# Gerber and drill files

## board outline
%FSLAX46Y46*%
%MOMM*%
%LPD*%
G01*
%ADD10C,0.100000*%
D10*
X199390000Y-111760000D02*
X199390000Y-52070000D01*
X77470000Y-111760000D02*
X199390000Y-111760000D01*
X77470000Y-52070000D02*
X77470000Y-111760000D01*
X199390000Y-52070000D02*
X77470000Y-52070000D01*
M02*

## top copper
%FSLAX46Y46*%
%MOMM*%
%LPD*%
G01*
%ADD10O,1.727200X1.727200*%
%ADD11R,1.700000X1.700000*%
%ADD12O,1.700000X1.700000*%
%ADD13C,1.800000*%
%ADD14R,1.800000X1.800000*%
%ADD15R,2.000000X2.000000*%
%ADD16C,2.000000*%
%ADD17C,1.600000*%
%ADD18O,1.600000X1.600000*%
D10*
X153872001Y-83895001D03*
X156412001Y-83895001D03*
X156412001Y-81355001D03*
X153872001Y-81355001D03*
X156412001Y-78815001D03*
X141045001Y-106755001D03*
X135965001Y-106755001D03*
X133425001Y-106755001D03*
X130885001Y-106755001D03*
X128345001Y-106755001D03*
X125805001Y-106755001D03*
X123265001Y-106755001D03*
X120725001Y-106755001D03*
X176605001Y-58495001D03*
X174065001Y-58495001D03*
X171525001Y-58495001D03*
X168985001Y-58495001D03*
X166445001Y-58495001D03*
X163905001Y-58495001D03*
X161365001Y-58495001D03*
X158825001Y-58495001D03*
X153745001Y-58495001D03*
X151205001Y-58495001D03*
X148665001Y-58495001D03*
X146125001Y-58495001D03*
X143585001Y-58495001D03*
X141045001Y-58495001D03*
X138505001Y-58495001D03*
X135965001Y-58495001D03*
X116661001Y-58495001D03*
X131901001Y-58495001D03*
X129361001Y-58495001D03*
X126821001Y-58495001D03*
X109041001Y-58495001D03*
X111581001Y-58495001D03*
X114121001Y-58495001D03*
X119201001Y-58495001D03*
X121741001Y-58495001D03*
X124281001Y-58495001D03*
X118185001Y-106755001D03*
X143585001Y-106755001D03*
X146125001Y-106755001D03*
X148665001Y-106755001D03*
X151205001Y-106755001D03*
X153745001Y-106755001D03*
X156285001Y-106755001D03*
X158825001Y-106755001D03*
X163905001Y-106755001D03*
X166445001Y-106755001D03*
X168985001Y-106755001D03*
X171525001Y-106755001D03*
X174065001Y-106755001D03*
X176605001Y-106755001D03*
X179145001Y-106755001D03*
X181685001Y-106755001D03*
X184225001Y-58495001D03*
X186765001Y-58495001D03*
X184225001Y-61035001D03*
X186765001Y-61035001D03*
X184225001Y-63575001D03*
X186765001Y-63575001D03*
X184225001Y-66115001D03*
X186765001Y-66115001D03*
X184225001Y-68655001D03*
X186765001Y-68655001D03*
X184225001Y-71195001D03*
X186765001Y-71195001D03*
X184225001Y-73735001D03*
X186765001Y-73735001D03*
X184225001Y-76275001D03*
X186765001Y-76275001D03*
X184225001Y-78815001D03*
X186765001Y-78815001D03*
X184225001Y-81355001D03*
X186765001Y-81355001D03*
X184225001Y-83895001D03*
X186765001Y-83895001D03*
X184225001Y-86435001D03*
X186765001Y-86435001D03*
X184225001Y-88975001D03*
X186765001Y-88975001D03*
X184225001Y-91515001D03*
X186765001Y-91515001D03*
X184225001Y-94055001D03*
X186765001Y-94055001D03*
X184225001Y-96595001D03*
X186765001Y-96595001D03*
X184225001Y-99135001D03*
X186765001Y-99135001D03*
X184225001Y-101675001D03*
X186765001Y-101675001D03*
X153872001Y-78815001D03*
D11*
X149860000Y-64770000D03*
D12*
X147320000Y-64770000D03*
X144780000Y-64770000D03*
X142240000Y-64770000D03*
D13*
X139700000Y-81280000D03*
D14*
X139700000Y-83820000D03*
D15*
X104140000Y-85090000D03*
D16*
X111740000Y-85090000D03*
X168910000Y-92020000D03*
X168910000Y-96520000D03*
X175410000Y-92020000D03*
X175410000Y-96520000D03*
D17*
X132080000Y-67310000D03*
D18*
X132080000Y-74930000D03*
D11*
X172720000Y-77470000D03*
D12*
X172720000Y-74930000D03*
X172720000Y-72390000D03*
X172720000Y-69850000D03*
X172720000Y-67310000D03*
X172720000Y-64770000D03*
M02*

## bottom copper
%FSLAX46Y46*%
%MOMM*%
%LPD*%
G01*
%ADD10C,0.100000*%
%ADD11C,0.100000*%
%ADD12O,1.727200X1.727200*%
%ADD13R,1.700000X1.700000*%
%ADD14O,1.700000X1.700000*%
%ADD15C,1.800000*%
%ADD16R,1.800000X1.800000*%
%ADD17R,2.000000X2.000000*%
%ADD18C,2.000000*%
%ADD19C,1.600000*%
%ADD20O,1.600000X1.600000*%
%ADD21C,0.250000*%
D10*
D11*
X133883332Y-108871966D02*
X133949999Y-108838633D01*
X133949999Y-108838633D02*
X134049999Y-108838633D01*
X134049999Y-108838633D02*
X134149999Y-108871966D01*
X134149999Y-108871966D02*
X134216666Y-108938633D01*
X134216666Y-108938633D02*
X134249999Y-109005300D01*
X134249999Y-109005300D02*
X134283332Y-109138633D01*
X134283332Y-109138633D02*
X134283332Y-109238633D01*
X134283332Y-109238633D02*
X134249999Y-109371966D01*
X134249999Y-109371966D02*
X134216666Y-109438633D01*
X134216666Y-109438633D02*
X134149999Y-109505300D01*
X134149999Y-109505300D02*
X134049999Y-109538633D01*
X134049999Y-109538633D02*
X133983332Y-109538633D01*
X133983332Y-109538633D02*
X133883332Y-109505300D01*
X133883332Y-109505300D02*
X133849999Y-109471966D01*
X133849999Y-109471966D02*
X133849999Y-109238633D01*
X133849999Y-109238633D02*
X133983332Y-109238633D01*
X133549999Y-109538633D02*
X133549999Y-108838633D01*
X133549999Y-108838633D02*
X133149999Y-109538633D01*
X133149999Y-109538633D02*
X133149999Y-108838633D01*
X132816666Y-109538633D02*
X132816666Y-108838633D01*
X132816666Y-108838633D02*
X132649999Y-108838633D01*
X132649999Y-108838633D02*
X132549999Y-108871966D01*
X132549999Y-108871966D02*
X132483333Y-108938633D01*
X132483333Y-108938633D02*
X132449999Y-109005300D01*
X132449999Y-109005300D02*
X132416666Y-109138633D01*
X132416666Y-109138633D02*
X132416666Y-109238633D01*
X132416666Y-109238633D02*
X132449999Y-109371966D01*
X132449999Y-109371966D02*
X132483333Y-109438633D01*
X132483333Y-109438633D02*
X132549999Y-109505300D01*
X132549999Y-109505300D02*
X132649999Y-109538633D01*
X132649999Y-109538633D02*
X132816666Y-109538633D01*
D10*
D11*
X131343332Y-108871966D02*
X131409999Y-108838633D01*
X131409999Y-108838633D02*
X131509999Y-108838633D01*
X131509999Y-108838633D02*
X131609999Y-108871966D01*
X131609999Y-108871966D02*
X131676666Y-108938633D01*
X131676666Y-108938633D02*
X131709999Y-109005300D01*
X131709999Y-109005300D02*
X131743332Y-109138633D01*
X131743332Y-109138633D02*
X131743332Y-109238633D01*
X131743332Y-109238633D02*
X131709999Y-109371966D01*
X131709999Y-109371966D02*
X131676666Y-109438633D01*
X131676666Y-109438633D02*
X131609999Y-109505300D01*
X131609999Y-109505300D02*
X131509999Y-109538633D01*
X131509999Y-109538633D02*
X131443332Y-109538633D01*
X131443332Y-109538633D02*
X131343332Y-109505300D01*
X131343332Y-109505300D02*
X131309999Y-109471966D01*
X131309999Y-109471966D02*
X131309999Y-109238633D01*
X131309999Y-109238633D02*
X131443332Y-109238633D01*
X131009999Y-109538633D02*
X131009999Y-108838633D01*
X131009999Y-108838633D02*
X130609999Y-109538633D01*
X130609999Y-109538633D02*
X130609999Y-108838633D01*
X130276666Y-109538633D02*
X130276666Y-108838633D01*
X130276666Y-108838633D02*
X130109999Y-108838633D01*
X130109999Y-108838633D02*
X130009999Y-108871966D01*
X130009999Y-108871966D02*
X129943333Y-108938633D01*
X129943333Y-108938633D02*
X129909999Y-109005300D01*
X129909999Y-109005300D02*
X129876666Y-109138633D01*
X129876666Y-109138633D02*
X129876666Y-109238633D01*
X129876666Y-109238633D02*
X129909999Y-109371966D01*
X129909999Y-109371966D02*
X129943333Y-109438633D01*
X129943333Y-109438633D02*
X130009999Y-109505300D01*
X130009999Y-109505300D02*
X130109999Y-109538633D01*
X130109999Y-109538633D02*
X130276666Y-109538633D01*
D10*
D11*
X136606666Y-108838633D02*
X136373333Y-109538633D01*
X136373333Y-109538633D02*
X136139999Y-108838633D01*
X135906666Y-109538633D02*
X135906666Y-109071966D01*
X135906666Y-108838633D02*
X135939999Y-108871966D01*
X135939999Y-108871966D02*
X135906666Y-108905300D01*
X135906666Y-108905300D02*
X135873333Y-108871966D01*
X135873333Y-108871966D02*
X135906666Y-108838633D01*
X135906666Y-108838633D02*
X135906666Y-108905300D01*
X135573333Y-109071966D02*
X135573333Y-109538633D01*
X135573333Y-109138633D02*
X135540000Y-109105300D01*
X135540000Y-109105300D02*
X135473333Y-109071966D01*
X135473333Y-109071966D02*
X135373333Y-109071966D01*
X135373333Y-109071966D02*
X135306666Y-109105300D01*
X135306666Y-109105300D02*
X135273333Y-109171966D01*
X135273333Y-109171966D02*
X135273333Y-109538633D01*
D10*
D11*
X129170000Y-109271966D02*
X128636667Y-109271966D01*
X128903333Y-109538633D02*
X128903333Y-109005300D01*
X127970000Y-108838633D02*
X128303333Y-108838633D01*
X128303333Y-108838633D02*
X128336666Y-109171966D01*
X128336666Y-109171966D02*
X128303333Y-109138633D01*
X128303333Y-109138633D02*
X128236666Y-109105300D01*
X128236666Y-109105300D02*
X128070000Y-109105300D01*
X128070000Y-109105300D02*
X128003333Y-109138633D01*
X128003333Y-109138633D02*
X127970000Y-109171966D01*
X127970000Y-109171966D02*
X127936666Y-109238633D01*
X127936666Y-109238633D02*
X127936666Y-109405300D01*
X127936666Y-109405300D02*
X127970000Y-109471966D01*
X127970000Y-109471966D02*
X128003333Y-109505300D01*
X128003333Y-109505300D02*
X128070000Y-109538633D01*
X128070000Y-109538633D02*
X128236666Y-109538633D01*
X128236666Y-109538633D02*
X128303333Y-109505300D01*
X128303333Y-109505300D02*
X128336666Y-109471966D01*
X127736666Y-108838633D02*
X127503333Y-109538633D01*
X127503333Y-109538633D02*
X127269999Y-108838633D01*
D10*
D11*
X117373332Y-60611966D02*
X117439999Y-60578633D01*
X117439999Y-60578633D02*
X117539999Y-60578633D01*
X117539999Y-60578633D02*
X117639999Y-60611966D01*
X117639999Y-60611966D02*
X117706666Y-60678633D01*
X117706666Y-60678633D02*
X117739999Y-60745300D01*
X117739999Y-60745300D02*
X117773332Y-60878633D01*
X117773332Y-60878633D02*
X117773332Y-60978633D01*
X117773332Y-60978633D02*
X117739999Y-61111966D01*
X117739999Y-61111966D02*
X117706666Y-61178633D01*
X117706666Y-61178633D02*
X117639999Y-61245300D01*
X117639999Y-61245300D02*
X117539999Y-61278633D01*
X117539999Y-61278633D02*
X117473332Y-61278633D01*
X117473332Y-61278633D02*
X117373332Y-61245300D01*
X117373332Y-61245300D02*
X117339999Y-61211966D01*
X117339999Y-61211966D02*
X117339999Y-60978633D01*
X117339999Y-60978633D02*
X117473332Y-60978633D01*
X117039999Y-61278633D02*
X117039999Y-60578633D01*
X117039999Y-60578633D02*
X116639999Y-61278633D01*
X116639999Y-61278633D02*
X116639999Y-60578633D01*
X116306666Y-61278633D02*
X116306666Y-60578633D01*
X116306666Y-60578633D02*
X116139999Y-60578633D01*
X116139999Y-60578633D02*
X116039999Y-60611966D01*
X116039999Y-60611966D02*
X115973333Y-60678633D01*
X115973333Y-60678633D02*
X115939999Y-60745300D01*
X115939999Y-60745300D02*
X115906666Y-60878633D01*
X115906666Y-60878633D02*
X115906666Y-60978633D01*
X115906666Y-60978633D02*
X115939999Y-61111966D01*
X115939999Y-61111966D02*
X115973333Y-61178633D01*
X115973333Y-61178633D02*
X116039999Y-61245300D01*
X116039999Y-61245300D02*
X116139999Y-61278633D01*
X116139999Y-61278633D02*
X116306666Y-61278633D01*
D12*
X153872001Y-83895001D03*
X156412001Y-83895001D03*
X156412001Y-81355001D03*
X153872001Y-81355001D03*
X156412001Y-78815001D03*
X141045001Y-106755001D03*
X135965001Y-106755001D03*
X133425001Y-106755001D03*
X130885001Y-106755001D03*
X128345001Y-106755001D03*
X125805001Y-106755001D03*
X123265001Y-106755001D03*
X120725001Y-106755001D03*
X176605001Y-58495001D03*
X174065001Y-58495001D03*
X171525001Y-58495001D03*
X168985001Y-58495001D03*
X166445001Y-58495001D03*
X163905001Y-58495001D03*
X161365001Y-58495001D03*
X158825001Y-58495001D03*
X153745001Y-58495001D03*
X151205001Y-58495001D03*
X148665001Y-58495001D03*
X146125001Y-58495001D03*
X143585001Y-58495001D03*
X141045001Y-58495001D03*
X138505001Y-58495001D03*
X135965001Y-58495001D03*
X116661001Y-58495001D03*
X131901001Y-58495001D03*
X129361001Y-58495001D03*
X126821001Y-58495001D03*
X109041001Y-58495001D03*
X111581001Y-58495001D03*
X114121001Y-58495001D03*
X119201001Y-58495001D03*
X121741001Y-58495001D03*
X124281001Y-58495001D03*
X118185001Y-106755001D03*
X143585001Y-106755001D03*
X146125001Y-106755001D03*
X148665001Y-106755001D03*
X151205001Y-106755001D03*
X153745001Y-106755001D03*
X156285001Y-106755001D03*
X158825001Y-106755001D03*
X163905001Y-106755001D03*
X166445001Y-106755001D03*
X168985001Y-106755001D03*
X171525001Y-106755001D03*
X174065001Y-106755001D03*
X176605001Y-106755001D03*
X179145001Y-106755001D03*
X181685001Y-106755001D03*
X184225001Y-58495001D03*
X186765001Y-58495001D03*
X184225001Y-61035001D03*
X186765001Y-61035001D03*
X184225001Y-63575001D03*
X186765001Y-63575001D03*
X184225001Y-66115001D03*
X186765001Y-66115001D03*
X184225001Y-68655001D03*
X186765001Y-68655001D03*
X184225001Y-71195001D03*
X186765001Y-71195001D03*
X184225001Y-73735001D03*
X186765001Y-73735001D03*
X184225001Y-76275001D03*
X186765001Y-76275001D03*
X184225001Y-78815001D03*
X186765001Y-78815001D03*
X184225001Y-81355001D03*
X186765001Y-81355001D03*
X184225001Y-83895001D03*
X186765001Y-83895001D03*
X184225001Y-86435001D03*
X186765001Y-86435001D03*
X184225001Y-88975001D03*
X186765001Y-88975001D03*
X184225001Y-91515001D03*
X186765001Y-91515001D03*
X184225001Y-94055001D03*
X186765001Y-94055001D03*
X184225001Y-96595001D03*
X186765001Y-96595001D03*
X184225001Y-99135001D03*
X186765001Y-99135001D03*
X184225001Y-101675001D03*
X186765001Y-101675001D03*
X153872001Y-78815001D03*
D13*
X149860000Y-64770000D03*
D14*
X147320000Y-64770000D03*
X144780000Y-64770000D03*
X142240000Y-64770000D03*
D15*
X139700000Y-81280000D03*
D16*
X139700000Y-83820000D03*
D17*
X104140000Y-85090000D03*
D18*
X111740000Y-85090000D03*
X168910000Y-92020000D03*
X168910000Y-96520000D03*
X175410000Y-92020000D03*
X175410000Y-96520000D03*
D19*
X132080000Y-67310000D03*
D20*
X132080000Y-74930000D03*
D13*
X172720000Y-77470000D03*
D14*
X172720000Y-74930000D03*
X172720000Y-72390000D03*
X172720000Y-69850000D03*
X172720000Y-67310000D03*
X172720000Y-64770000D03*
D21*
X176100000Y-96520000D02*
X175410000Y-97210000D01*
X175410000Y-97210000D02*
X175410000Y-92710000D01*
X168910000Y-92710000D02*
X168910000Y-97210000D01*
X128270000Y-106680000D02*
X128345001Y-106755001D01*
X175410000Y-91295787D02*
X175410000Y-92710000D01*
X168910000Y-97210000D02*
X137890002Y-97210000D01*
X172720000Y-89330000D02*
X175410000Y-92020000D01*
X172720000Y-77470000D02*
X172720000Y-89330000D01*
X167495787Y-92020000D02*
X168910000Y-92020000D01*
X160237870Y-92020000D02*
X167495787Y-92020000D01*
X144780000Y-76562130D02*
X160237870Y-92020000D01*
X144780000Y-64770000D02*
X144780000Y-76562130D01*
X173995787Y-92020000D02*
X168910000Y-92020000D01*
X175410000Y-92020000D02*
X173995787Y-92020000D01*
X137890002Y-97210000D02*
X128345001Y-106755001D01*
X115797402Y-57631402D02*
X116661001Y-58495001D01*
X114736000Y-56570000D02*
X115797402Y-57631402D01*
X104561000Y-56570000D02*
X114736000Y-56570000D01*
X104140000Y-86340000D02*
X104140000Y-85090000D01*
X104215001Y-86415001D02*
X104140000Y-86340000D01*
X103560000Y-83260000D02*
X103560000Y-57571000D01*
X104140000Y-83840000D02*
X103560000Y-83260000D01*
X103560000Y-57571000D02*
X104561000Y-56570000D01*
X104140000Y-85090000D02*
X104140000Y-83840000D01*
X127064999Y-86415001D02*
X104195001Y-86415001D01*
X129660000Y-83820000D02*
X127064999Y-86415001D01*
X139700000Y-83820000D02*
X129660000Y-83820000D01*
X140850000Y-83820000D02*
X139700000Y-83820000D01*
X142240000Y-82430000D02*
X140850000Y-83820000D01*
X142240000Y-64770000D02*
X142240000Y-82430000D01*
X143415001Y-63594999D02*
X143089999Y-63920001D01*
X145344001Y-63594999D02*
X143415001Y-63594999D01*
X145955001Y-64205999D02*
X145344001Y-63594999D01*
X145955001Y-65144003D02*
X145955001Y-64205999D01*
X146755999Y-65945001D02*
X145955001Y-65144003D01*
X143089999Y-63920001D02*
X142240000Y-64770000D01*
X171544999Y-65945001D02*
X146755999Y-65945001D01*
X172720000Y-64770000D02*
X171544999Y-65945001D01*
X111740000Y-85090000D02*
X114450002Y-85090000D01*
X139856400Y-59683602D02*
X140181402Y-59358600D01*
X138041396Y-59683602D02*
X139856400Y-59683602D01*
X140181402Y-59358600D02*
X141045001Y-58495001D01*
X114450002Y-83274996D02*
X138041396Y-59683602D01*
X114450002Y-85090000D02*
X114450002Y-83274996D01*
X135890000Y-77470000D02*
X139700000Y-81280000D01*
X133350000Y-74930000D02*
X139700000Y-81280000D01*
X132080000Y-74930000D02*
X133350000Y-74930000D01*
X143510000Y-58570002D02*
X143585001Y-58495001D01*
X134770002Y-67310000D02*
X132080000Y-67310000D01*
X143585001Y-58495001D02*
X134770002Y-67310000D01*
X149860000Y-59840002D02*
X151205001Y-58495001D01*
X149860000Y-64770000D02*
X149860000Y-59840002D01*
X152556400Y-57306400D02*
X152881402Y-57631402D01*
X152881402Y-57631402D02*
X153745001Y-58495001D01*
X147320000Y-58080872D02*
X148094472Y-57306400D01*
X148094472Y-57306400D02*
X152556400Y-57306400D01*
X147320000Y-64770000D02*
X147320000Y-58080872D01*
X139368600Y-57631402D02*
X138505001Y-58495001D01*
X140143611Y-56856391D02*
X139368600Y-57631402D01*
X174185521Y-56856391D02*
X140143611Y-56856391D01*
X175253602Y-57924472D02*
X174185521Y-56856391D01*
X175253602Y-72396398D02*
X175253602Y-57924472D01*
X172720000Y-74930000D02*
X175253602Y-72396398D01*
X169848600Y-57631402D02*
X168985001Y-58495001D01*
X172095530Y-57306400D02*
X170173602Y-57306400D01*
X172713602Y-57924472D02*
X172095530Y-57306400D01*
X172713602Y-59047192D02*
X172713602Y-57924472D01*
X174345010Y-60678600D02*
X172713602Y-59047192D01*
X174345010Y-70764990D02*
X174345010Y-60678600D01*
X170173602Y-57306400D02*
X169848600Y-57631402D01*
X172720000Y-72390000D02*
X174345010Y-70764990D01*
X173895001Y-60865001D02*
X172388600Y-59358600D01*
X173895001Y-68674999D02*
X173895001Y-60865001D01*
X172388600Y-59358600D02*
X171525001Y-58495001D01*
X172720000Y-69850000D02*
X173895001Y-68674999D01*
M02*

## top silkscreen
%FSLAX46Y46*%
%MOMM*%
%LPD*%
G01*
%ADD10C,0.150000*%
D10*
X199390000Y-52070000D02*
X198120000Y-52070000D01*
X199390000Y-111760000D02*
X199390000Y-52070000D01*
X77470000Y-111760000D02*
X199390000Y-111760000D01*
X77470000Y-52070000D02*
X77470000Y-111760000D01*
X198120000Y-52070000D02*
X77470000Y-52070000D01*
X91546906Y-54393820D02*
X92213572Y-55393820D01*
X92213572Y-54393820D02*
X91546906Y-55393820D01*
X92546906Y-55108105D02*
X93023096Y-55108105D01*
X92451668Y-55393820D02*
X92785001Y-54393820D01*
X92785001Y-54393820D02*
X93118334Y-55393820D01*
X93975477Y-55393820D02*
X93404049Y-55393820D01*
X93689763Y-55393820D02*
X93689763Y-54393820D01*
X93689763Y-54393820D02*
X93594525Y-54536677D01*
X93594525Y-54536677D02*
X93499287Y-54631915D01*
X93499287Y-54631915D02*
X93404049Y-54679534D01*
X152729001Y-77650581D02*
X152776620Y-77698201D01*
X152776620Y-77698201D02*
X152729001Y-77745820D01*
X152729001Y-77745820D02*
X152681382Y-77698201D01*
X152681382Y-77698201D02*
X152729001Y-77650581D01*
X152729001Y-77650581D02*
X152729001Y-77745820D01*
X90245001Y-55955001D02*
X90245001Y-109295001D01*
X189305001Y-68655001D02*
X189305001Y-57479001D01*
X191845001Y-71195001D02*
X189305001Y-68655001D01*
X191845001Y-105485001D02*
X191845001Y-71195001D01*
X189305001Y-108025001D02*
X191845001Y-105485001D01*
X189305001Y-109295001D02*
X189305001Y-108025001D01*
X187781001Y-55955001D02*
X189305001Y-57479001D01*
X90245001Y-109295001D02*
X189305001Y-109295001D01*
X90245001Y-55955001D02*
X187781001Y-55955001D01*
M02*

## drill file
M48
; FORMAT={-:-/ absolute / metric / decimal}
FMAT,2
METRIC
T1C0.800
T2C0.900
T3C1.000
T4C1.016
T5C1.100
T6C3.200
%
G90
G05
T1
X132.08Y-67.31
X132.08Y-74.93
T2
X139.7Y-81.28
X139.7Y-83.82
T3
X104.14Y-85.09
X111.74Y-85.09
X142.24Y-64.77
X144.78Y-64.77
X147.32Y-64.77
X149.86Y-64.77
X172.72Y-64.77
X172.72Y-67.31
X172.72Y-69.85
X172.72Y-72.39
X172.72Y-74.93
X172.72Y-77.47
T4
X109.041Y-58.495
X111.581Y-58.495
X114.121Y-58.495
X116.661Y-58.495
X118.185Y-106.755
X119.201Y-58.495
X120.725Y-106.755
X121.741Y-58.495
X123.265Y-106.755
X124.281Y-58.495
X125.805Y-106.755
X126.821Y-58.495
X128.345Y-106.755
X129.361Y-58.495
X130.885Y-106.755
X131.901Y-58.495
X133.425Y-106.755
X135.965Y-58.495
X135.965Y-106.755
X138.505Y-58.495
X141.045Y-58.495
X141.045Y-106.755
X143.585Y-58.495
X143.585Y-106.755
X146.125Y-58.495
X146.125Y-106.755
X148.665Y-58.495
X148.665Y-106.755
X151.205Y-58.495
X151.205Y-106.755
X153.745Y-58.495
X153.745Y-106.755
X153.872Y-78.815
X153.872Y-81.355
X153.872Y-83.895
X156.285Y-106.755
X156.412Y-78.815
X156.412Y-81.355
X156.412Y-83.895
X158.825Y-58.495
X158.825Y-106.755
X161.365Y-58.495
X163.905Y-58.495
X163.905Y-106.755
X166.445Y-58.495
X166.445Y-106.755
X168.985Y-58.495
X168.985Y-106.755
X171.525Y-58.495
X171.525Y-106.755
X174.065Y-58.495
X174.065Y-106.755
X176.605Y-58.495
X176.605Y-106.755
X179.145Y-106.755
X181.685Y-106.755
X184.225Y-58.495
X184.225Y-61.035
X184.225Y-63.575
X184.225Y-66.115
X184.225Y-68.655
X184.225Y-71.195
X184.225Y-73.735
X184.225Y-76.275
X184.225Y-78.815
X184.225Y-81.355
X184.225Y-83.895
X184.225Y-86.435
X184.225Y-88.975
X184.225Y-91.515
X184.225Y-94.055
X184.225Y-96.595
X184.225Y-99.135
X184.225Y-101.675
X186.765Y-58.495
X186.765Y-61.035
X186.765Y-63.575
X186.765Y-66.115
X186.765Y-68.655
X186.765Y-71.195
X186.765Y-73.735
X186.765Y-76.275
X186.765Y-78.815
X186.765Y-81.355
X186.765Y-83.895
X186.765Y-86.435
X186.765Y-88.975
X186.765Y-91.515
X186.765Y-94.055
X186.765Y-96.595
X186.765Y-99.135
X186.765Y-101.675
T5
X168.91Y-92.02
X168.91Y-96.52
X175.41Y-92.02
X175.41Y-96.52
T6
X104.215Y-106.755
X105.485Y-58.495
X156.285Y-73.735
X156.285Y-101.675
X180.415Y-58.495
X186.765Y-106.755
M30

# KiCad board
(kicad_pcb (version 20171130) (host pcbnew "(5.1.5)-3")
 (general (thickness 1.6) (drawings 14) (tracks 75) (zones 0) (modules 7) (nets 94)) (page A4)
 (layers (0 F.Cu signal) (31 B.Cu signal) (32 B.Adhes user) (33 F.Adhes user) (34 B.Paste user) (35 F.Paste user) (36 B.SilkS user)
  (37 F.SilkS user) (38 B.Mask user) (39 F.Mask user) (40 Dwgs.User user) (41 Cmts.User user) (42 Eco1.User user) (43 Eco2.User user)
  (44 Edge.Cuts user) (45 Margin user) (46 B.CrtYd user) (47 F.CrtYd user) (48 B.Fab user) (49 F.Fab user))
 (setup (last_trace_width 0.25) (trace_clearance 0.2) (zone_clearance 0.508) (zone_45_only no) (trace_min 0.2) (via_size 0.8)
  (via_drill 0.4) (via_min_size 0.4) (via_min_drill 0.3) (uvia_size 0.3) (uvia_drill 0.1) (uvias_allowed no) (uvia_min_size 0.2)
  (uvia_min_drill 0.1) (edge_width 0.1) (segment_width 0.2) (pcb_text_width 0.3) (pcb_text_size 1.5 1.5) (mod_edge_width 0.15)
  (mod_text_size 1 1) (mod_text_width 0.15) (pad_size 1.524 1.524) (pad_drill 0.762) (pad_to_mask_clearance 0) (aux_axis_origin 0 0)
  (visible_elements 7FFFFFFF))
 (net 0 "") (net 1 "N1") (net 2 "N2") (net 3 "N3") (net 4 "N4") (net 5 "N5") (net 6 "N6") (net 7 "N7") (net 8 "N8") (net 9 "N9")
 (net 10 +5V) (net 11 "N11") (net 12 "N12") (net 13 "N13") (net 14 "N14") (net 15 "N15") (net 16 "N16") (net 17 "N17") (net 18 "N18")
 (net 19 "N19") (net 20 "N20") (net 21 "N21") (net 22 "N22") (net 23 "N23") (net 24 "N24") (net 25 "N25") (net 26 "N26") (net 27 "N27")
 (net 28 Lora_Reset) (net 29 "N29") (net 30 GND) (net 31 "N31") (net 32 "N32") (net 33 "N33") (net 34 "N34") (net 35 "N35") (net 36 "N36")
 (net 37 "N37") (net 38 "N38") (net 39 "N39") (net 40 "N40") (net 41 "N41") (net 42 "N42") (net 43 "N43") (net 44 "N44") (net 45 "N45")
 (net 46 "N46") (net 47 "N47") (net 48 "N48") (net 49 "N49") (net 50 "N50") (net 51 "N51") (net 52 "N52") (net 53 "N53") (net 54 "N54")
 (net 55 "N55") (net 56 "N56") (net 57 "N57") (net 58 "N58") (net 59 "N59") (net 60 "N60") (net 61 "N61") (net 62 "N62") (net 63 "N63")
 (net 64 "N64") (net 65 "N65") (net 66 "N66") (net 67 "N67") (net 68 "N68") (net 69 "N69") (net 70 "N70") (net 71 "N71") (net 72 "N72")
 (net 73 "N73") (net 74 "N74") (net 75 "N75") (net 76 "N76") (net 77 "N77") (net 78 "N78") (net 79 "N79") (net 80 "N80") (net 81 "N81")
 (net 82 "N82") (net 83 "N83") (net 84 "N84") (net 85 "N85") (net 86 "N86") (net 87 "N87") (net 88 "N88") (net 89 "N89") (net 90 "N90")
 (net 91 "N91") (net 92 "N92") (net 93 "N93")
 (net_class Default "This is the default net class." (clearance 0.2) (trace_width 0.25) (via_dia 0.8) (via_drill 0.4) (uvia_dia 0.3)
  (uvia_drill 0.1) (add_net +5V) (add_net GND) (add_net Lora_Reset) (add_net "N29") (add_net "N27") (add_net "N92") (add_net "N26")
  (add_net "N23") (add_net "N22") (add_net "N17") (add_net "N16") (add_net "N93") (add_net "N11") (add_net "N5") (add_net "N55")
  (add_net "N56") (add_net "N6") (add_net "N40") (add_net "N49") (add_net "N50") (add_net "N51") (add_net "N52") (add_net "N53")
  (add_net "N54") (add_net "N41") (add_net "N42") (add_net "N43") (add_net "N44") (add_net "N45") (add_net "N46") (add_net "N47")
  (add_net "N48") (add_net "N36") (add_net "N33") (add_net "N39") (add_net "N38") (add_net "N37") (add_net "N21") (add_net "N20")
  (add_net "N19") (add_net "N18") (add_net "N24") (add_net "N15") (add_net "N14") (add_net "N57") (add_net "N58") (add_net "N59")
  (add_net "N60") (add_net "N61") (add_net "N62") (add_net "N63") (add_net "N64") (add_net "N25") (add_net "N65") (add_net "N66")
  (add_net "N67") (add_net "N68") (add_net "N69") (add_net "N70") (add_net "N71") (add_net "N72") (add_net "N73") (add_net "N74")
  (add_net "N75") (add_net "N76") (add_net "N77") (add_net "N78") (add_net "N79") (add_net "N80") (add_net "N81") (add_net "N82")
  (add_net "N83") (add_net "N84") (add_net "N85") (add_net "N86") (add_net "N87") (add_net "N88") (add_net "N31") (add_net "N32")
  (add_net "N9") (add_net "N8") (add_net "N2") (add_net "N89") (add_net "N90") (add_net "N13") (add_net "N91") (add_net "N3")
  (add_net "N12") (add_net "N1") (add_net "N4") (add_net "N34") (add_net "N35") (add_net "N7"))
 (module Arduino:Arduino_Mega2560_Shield (layer F.Cu) (at 90.245001 109.295001)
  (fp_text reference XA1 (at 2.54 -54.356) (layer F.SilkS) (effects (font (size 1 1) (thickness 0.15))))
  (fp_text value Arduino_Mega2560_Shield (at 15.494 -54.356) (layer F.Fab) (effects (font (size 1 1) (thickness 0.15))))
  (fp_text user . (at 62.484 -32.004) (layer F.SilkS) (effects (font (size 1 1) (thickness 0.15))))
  (fp_line (start 0 -53.34) (end 0 0) (layer F.SilkS) (width 0.15))
  (fp_line (start 99.06 -40.64) (end 99.06 -51.816) (layer F.SilkS) (width 0.15))
  (fp_line (start 101.6 -38.1) (end 99.06 -40.64) (layer F.SilkS) (width 0.15))
  (fp_line (start 101.6 -3.81) (end 101.6 -38.1) (layer F.SilkS) (width 0.15))
  (fp_line (start 99.06 -1.27) (end 101.6 -3.81) (layer F.SilkS) (width 0.15))
  (fp_line (start 99.06 0) (end 99.06 -1.27) (layer F.SilkS) (width 0.15))
  (fp_line (start 97.536 -53.34) (end 99.06 -51.816) (layer F.SilkS) (width 0.15))
  (fp_line (start 0 0) (end 99.06 0) (layer F.SilkS) (width 0.15))
  (fp_line (start 0 -53.34) (end 97.536 -53.34) (layer F.SilkS) (width 0.15))
  (pad RST2 thru_hole oval (at 63.627 -25.4) (size 1.7272 1.7272) (drill 1.016) (layers *.Cu *.Mask) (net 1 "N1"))
  (pad GND4 thru_hole oval (at 66.167 -25.4) (size 1.7272 1.7272) (drill 1.016) (layers *.Cu *.Mask) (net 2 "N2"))
  (pad MOSI thru_hole oval (at 66.167 -27.94) (size 1.7272 1.7272) (drill 1.016) (layers *.Cu *.Mask) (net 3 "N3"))
  (pad SCK thru_hole oval (at 63.627 -27.94) (size 1.7272 1.7272) (drill 1.016) (layers *.Cu *.Mask) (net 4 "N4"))
  (pad 5V2 thru_hole oval (at 66.167 -30.48) (size 1.7272 1.7272) (drill 1.016) (layers *.Cu *.Mask) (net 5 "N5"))
  (pad A0 thru_hole oval (at 50.8 -2.54) (size 1.7272 1.7272) (drill 1.016) (layers *.Cu *.Mask) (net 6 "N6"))
  (pad VIN thru_hole oval (at 45.72 -2.54) (size 1.7272 1.7272) (drill 1.016) (layers *.Cu *.Mask) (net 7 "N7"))
  (pad GND3 thru_hole oval (at 43.18 -2.54) (size 1.7272 1.7272) (drill 1.016) (layers *.Cu *.Mask) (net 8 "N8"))
  (pad GND2 thru_hole oval (at 40.64 -2.54) (size 1.7272 1.7272) (drill 1.016) (layers *.Cu *.Mask) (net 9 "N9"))
  (pad 5V1 thru_hole oval (at 38.1 -2.54) (size 1.7272 1.7272) (drill 1.016) (layers *.Cu *.Mask) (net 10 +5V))
  (pad 3V3 thru_hole oval (at 35.56 -2.54) (size 1.7272 1.7272) (drill 1.016) (layers *.Cu *.Mask) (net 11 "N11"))
  (pad RST1 thru_hole oval (at 33.02 -2.54) (size 1.7272 1.7272) (drill 1.016) (layers *.Cu *.Mask) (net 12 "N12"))
  (pad IORF thru_hole oval (at 30.48 -2.54) (size 1.7272 1.7272) (drill 1.016) (layers *.Cu *.Mask) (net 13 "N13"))
  (pad D21 thru_hole oval (at 86.36 -50.8) (size 1.7272 1.7272) (drill 1.016) (layers *.Cu *.Mask) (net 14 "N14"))
  (pad D20 thru_hole oval (at 83.82 -50.8) (size 1.7272 1.7272) (drill 1.016) (layers *.Cu *.Mask) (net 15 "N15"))
  (pad D19 thru_hole oval (at 81.28 -50.8) (size 1.7272 1.7272) (drill 1.016) (layers *.Cu *.Mask) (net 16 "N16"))
  (pad D18 thru_hole oval (at 78.74 -50.8) (size 1.7272 1.7272) (drill 1.016) (layers *.Cu *.Mask) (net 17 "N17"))
  (pad D17 thru_hole oval (at 76.2 -50.8) (size 1.7272 1.7272) (drill 1.016) (layers *.Cu *.Mask) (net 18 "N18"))
  (pad D16 thru_hole oval (at 73.66 -50.8) (size 1.7272 1.7272) (drill 1.016) (layers *.Cu *.Mask) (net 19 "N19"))
  (pad D15 thru_hole oval (at 71.12 -50.8) (size 1.7272 1.7272) (drill 1.016) (layers *.Cu *.Mask) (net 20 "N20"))
  (pad D14 thru_hole oval (at 68.58 -50.8) (size 1.7272 1.7272) (drill 1.016) (layers *.Cu *.Mask) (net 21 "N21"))
  (pad D0 thru_hole oval (at 63.5 -50.8) (size 1.7272 1.7272) (drill 1.016) (layers *.Cu *.Mask) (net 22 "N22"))
  (pad D1 thru_hole oval (at 60.96 -50.8) (size 1.7272 1.7272) (drill 1.016) (layers *.Cu *.Mask) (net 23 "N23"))
  (pad D2 thru_hole oval (at 58.42 -50.8) (size 1.7272 1.7272) (drill 1.016) (layers *.Cu *.Mask) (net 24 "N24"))
  (pad D3 thru_hole oval (at 55.88 -50.8) (size 1.7272 1.7272) (drill 1.016) (layers *.Cu *.Mask) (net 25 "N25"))
  (pad D4 thru_hole oval (at 53.34 -50.8) (size 1.7272 1.7272) (drill 1.016) (layers *.Cu *.Mask) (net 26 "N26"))
  (pad D5 thru_hole oval (at 50.8 -50.8) (size 1.7272 1.7272) (drill 1.016) (layers *.Cu *.Mask) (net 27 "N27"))
  (pad D6 thru_hole oval (at 48.26 -50.8) (size 1.7272 1.7272) (drill 1.016) (layers *.Cu *.Mask) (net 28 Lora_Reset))
  (pad D7 thru_hole oval (at 45.72 -50.8) (size 1.7272 1.7272) (drill 1.016) (layers *.Cu *.Mask) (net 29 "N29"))
  (pad GND1 thru_hole oval (at 26.416 -50.8) (size 1.7272 1.7272) (drill 1.016) (layers *.Cu *.Mask) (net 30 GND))
  (pad D8 thru_hole oval (at 41.656 -50.8) (size 1.7272 1.7272) (drill 1.016) (layers *.Cu *.Mask) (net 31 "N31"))
  (pad D9 thru_hole oval (at 39.116 -50.8) (size 1.7272 1.7272) (drill 1.016) (layers *.Cu *.Mask) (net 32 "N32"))
  (pad D10 thru_hole oval (at 36.576 -50.8) (size 1.7272 1.7272) (drill 1.016) (layers *.Cu *.Mask) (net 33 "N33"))
  (pad "" np_thru_hole circle (at 66.04 -7.62) (size 3.2 3.2) (drill 3.2) (layers *.Cu *.Mask))
  (pad "" np_thru_hole circle (at 66.04 -35.56) (size 3.2 3.2) (drill 3.2) (layers *.Cu *.Mask))
  (pad "" np_thru_hole circle (at 90.17 -50.8) (size 3.2 3.2) (drill 3.2) (layers *.Cu *.Mask))
  (pad "" np_thru_hole circle (at 15.24 -50.8) (size 3.2 3.2) (drill 3.2) (layers *.Cu *.Mask))
  (pad "" np_thru_hole circle (at 96.52 -2.54) (size 3.2 3.2) (drill 3.2) (layers *.Cu *.Mask))
  (pad "" np_thru_hole circle (at 13.97 -2.54) (size 3.2 3.2) (drill 3.2) (layers *.Cu *.Mask))
  (pad SCL thru_hole oval (at 18.796 -50.8) (size 1.7272 1.7272) (drill 1.016) (layers *.Cu *.Mask) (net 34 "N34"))
  (pad SDA thru_hole oval (at 21.336 -50.8) (size 1.7272 1.7272) (drill 1.016) (layers *.Cu *.Mask) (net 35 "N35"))
  (pad AREF thru_hole oval (at 23.876 -50.8) (size 1.7272 1.7272) (drill 1.016) (layers *.Cu *.Mask) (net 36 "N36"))
  (pad D13 thru_hole oval (at 28.956 -50.8) (size 1.7272 1.7272) (drill 1.016) (layers *.Cu *.Mask) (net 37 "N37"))
  (pad D12 thru_hole oval (at 31.496 -50.8) (size 1.7272 1.7272) (drill 1.016) (layers *.Cu *.Mask) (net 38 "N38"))
  (pad D11 thru_hole oval (at 34.036 -50.8) (size 1.7272 1.7272) (drill 1.016) (layers *.Cu *.Mask) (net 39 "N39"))
  (pad "" thru_hole oval (at 27.94 -2.54) (size 1.7272 1.7272) (drill 1.016) (layers *.Cu *.Mask))
  (pad A1 thru_hole oval (at 53.34 -2.54) (size 1.7272 1.7272) (drill 1.016) (layers *.Cu *.Mask) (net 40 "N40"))
  (pad A2 thru_hole oval (at 55.88 -2.54) (size 1.7272 1.7272) (drill 1.016) (layers *.Cu *.Mask) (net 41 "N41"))
  (pad A3 thru_hole oval (at 58.42 -2.54) (size 1.7272 1.7272) (drill 1.016) (layers *.Cu *.Mask) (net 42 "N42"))
  (pad A4 thru_hole oval (at 60.96 -2.54) (size 1.7272 1.7272) (drill 1.016) (layers *.Cu *.Mask) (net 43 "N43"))
  (pad A5 thru_hole oval (at 63.5 -2.54) (size 1.7272 1.7272) (drill 1.016) (layers *.Cu *.Mask) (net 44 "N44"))
  (pad A6 thru_hole oval (at 66.04 -2.54) (size 1.7272 1.7272) (drill 1.016) (layers *.Cu *.Mask) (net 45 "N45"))
  (pad A7 thru_hole oval (at 68.58 -2.54) (size 1.7272 1.7272) (drill 1.016) (layers *.Cu *.Mask) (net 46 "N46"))
  (pad A8 thru_hole oval (at 73.66 -2.54) (size 1.7272 1.7272) (drill 1.016) (layers *.Cu *.Mask) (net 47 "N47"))
  (pad A9 thru_hole oval (at 76.2 -2.54) (size 1.7272 1.7272) (drill 1.016) (layers *.Cu *.Mask) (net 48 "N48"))
  (pad A10 thru_hole oval (at 78.74 -2.54) (size 1.7272 1.7272) (drill 1.016) (layers *.Cu *.Mask) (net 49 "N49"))
  (pad A11 thru_hole oval (at 81.28 -2.54) (size 1.7272 1.7272) (drill 1.016) (layers *.Cu *.Mask) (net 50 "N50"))
  (pad A12 thru_hole oval (at 83.82 -2.54) (size 1.7272 1.7272) (drill 1.016) (layers *.Cu *.Mask) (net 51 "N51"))
  (pad A13 thru_hole oval (at 86.36 -2.54) (size 1.7272 1.7272) (drill 1.016) (layers *.Cu *.Mask) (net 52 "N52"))
  (pad A14 thru_hole oval (at 88.9 -2.54) (size 1.7272 1.7272) (drill 1.016) (layers *.Cu *.Mask) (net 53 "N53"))
  (pad A15 thru_hole oval (at 91.44 -2.54) (size 1.7272 1.7272) (drill 1.016) (layers *.Cu *.Mask) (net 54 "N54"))
  (pad 5V3 thru_hole oval (at 93.98 -50.8) (size 1.7272 1.7272) (drill 1.016) (layers *.Cu *.Mask) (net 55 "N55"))
  (pad 5V4 thru_hole oval (at 96.52 -50.8) (size 1.7272 1.7272) (drill 1.016) (layers *.Cu *.Mask) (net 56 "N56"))
  (pad D22 thru_hole oval (at 93.98 -48.26) (size 1.7272 1.7272) (drill 1.016) (layers *.Cu *.Mask) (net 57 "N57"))
  (pad D23 thru_hole oval (at 96.52 -48.26) (size 1.7272 1.7272) (drill 1.016) (layers *.Cu *.Mask) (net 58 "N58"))
  (pad D24 thru_hole oval (at 93.98 -45.72) (size 1.7272 1.7272) (drill 1.016) (layers *.Cu *.Mask) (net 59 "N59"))
  (pad D25 thru_hole oval (at 96.52 -45.72) (size 1.7272 1.7272) (drill 1.016) (layers *.Cu *.Mask) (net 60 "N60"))
  (pad D26 thru_hole oval (at 93.98 -43.18) (size 1.7272 1.7272) (drill 1.016) (layers *.Cu *.Mask) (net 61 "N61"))
  (pad D27 thru_hole oval (at 96.52 -43.18) (size 1.7272 1.7272) (drill 1.016) (layers *.Cu *.Mask) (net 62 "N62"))
  (pad D28 thru_hole oval (at 93.98 -40.64) (size 1.7272 1.7272) (drill 1.016) (layers *.Cu *.Mask) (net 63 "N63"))
  (pad D29 thru_hole oval (at 96.52 -40.64) (size 1.7272 1.7272) (drill 1.016) (layers *.Cu *.Mask) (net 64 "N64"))
  (pad D30 thru_hole oval (at 93.98 -38.1) (size 1.7272 1.7272) (drill 1.016) (layers *.Cu *.Mask) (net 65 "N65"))
  (pad D31 thru_hole oval (at 96.52 -38.1) (size 1.7272 1.7272) (drill 1.016) (layers *.Cu *.Mask) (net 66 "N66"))
  (pad D32 thru_hole oval (at 93.98 -35.56) (size 1.7272 1.7272) (drill 1.016) (layers *.Cu *.Mask) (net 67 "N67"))
  (pad D33 thru_hole oval (at 96.52 -35.56) (size 1.7272 1.7272) (drill 1.016) (layers *.Cu *.Mask) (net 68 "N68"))
  (pad D34 thru_hole oval (at 93.98 -33.02) (size 1.7272 1.7272) (drill 1.016) (layers *.Cu *.Mask) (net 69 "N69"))
  (pad D35 thru_hole oval (at 96.52 -33.02) (size 1.7272 1.7272) (drill 1.016) (layers *.Cu *.Mask) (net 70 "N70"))
  (pad D36 thru_hole oval (at 93.98 -30.48) (size 1.7272 1.7272) (drill 1.016) (layers *.Cu *.Mask) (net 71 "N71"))
  (pad D37 thru_hole oval (at 96.52 -30.48) (size 1.7272 1.7272) (drill 1.016) (layers *.Cu *.Mask) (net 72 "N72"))
  (pad D38 thru_hole oval (at 93.98 -27.94) (size 1.7272 1.7272) (drill 1.016) (layers *.Cu *.Mask) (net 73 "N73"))
  (pad D39 thru_hole oval (at 96.52 -27.94) (size 1.7272 1.7272) (drill 1.016) (layers *.Cu *.Mask) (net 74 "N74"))
  (pad D40 thru_hole oval (at 93.98 -25.4) (size 1.7272 1.7272) (drill 1.016) (layers *.Cu *.Mask) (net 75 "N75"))
  (pad D41 thru_hole oval (at 96.52 -25.4) (size 1.7272 1.7272) (drill 1.016) (layers *.Cu *.Mask) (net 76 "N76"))
  (pad D42 thru_hole oval (at 93.98 -22.86) (size 1.7272 1.7272) (drill 1.016) (layers *.Cu *.Mask) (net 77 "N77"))
  (pad D43 thru_hole oval (at 96.52 -22.86) (size 1.7272 1.7272) (drill 1.016) (layers *.Cu *.Mask) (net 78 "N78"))
  (pad D44 thru_hole oval (at 93.98 -20.32) (size 1.7272 1.7272) (drill 1.016) (layers *.Cu *.Mask) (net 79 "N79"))
  (pad D45 thru_hole oval (at 96.52 -20.32) (size 1.7272 1.7272) (drill 1.016) (layers *.Cu *.Mask) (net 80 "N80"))
  (pad D46 thru_hole oval (at 93.98 -17.78) (size 1.7272 1.7272) (drill 1.016) (layers *.Cu *.Mask) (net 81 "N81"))
  (pad D47 thru_hole oval (at 96.52 -17.78) (size 1.7272 1.7272) (drill 1.016) (layers *.Cu *.Mask) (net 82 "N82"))
  (pad D48 thru_hole oval (at 93.98 -15.24) (size 1.7272 1.7272) (drill 1.016) (layers *.Cu *.Mask) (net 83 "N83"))
  (pad D49 thru_hole oval (at 96.52 -15.24) (size 1.7272 1.7272) (drill 1.016) (layers *.Cu *.Mask) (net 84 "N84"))
  (pad D50 thru_hole oval (at 93.98 -12.7) (size 1.7272 1.7272) (drill 1.016) (layers *.Cu *.Mask) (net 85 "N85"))
  (pad D51 thru_hole oval (at 96.52 -12.7) (size 1.7272 1.7272) (drill 1.016) (layers *.Cu *.Mask) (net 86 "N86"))
  (pad D52 thru_hole oval (at 93.98 -10.16) (size 1.7272 1.7272) (drill 1.016) (layers *.Cu *.Mask) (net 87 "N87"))
  (pad D53 thru_hole oval (at 96.52 -10.16) (size 1.7272 1.7272) (drill 1.016) (layers *.Cu *.Mask) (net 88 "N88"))
  (pad GND5 thru_hole oval (at 93.98 -7.62) (size 1.7272 1.7272) (drill 1.016) (layers *.Cu *.Mask) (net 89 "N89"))
  (pad GND6 thru_hole oval (at 96.52 -7.62) (size 1.7272 1.7272) (drill 1.016) (layers *.Cu *.Mask) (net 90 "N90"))
  (pad MISO thru_hole oval (at 63.627 -30.48) (size 1.7272 1.7272) (drill 1.016) (layers *.Cu *.Mask) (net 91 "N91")))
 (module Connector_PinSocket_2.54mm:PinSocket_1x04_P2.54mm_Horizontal (layer B.Cu) (at 149.86 64.77 90)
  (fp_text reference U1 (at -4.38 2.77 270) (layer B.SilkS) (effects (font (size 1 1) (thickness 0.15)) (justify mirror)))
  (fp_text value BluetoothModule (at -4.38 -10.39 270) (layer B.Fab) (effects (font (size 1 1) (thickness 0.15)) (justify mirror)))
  (pad 1 thru_hole rect (at 0 0 90) (size 1.7 1.7) (drill 1) (layers *.Cu *.Mask) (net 23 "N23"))
  (pad 2 thru_hole oval (at 0 -2.54 90) (size 1.7 1.7) (drill 1) (layers *.Cu *.Mask) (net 22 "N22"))
  (pad 3 thru_hole oval (at 0 -5.08 90) (size 1.7 1.7) (drill 1) (layers *.Cu *.Mask) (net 10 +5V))
  (pad 4 thru_hole oval (at 0 -7.62 90) (size 1.7 1.7) (drill 1) (layers *.Cu *.Mask) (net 30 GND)))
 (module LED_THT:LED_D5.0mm (layer B.Cu) (at 139.7 83.82 90)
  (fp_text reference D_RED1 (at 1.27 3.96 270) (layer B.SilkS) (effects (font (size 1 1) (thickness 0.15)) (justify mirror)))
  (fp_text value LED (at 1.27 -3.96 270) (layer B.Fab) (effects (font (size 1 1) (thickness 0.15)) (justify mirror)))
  (pad 2 thru_hole circle (at 2.54 0 90) (size 1.8 1.8) (drill 0.9) (layers *.Cu *.Mask) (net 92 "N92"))
  (pad 1 thru_hole rect (at 0 0 90) (size 1.8 1.8) (drill 0.9) (layers *.Cu *.Mask) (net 30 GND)))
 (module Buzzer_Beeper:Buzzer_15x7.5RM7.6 (layer B.Cu) (at 104.14 85.09)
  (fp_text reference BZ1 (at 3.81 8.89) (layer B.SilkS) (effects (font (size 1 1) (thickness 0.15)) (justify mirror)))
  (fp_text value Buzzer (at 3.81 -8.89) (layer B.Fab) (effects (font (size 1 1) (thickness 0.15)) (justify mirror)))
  (pad 1 thru_hole rect (at 0 0) (size 2 2) (drill 1) (layers *.Cu *.Mask) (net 30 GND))
  (pad 2 thru_hole circle (at 7.6 0) (size 2 2) (drill 1) (layers *.Cu *.Mask) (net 27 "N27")))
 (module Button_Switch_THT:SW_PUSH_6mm (layer B.Cu) (at 168.91 96.52)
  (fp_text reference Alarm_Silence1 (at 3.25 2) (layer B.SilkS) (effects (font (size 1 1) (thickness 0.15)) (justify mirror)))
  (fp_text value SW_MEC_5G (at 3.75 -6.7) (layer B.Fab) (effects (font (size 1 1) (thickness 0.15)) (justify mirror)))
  (pad 2 thru_hole circle (at 0 -4.5 270) (size 2 2) (drill 1.1) (layers *.Cu *.Mask) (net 10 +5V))
  (pad 1 thru_hole circle (at 0 0 270) (size 2 2) (drill 1.1) (layers *.Cu *.Mask) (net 10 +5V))
  (pad 2 thru_hole circle (at 6.5 -4.5 270) (size 2 2) (drill 1.1) (layers *.Cu *.Mask) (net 10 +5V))
  (pad 1 thru_hole circle (at 6.5 0 270) (size 2 2) (drill 1.1) (layers *.Cu *.Mask) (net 10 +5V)))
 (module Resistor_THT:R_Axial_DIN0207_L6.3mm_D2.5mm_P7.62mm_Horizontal (layer B.Cu) (at 132.08 67.31 270)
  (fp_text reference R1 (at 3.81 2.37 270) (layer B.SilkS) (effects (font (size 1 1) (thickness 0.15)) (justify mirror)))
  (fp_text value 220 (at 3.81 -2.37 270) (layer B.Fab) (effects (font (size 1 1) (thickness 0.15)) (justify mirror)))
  (pad 1 thru_hole circle (at 0 0 270) (size 1.6 1.6) (drill 0.8) (layers *.Cu *.Mask) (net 26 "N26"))
  (pad 2 thru_hole oval (at 7.62 0 270) (size 1.6 1.6) (drill 0.8) (layers *.Cu *.Mask) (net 92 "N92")))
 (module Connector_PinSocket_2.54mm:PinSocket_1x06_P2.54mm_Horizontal (layer B.Cu) (at 172.72 77.47)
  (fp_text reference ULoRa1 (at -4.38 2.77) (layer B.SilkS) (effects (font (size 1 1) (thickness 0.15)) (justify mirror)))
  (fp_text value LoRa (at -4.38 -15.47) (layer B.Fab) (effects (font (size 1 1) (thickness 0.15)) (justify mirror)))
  (pad 1 thru_hole rect (at 0 0) (size 1.7 1.7) (drill 1) (layers *.Cu *.Mask) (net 10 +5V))
  (pad 2 thru_hole oval (at 0 -2.54) (size 1.7 1.7) (drill 1) (layers *.Cu *.Mask) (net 28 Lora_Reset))
  (pad 3 thru_hole oval (at 0 -5.08) (size 1.7 1.7) (drill 1) (layers *.Cu *.Mask) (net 17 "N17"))
  (pad 4 thru_hole oval (at 0 -7.62) (size 1.7 1.7) (drill 1) (layers *.Cu *.Mask) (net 16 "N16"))
  (pad 5 thru_hole oval (at 0 -10.16) (size 1.7 1.7) (drill 1) (layers *.Cu *.Mask) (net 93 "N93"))
  (pad 6 thru_hole oval (at 0 -12.7) (size 1.7 1.7) (drill 1) (layers *.Cu *.Mask) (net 30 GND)))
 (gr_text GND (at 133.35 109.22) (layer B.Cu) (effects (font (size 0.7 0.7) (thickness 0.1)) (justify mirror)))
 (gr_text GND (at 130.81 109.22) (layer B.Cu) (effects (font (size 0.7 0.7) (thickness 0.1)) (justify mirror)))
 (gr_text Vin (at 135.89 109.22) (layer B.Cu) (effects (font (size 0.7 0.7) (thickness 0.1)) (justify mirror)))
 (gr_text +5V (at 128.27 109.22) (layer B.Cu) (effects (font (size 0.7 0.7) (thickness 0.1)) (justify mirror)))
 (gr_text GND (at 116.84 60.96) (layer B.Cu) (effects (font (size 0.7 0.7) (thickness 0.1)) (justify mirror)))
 (gr_line (start 199.39 111.76) (end 199.39 52.07) (layer Edge.Cuts) (width 0.1))
 (gr_line (start 77.47 111.76) (end 199.39 111.76) (layer Edge.Cuts) (width 0.1))
 (gr_line (start 77.47 52.07) (end 77.47 111.76) (layer Edge.Cuts) (width 0.1))
 (gr_line (start 199.39 52.07) (end 77.47 52.07) (layer Edge.Cuts) (width 0.1))
 (gr_line (start 199.39 52.07) (end 198.12 52.07) (layer F.SilkS) (width 0.15))
 (gr_line (start 199.39 111.76) (end 199.39 52.07) (layer F.SilkS) (width 0.15))
 (gr_line (start 77.47 111.76) (end 199.39 111.76) (layer F.SilkS) (width 0.15))
 (gr_line (start 77.47 52.07) (end 77.47 111.76) (layer F.SilkS) (width 0.15))
 (gr_line (start 198.12 52.07) (end 77.47 52.07) (layer F.SilkS) (width 0.15))
 (segment (start 176.1 96.52) (end 175.41 97.21) (width 0.25) (layer B.Cu) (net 10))
 (segment (start 175.41 97.21) (end 175.41 92.71) (width 0.25) (layer B.Cu) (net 10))
 (segment (start 168.91 92.71) (end 168.91 97.21) (width 0.25) (layer B.Cu) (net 10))
 (segment (start 128.27 106.68) (end 128.345001 106.755001) (width 0.25) (layer B.Cu) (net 10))
 (segment (start 175.41 91.295787) (end 175.41 92.71) (width 0.25) (layer B.Cu) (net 10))
 (segment (start 168.91 97.21) (end 137.890002 97.21) (width 0.25) (layer B.Cu) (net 10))
 (segment (start 172.72 89.33) (end 175.41 92.02) (width 0.25) (layer B.Cu) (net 10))
 (segment (start 172.72 77.47) (end 172.72 89.33) (width 0.25) (layer B.Cu) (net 10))
 (segment (start 167.495787 92.02) (end 168.91 92.02) (width 0.25) (layer B.Cu) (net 10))
 (segment (start 160.23787 92.02) (end 167.495787 92.02) (width 0.25) (layer B.Cu) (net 10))
 (segment (start 144.78 76.56213) (end 160.23787 92.02) (width 0.25) (layer B.Cu) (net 10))
 (segment (start 144.78 64.77) (end 144.78 76.56213) (width 0.25) (layer B.Cu) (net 10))
 (segment (start 173.995787 92.02) (end 168.91 92.02) (width 0.25) (layer B.Cu) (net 10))
 (segment (start 175.41 92.02) (end 173.995787 92.02) (width 0.25) (layer B.Cu) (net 10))
 (segment (start 137.890002 97.21) (end 128.345001 106.755001) (width 0.25) (layer B.Cu) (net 10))
 (segment (start 115.797402 57.631402) (end 116.661001 58.495001) (width 0.25) (layer B.Cu) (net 30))
 (segment (start 114.736 56.57) (end 115.797402 57.631402) (width 0.25) (layer B.Cu) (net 30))
 (segment (start 104.561 56.57) (end 114.736 56.57) (width 0.25) (layer B.Cu) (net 30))
 (segment (start 104.14 86.34) (end 104.14 85.09) (width 0.25) (layer B.Cu) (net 30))
 (segment (start 104.215001 86.415001) (end 104.14 86.34) (width 0.25) (layer B.Cu) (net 30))
 (segment (start 103.56 83.26) (end 103.56 57.571) (width 0.25) (layer B.Cu) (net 30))
 (segment (start 104.14 83.84) (end 103.56 83.26) (width 0.25) (layer B.Cu) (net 30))
 (segment (start 103.56 57.571) (end 104.561 56.57) (width 0.25) (layer B.Cu) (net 30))
 (segment (start 104.14 85.09) (end 104.14 83.84) (width 0.25) (layer B.Cu) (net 30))
 (segment (start 127.064999 86.415001) (end 104.195001 86.415001) (width 0.25) (layer B.Cu) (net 30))
 (segment (start 129.66 83.82) (end 127.064999 86.415001) (width 0.25) (layer B.Cu) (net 30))
 (segment (start 139.7 83.82) (end 129.66 83.82) (width 0.25) (layer B.Cu) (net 30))
 (segment (start 140.85 83.82) (end 139.7 83.82) (width 0.25) (layer B.Cu) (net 30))
 (segment (start 142.24 82.43) (end 140.85 83.82) (width 0.25) (layer B.Cu) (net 30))
 (segment (start 142.24 64.77) (end 142.24 82.43) (width 0.25) (layer B.Cu) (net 30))
 (segment (start 143.415001 63.594999) (end 143.089999 63.920001) (width 0.25) (layer B.Cu) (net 30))
 (segment (start 145.344001 63.594999) (end 143.415001 63.594999) (width 0.25) (layer B.Cu) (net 30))
 (segment (start 145.955001 64.205999) (end 145.344001 63.594999) (width 0.25) (layer B.Cu) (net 30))
 (segment (start 145.955001 65.144003) (end 145.955001 64.205999) (width 0.25) (layer B.Cu) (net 30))
 (segment (start 146.755999 65.945001) (end 145.955001 65.144003) (width 0.25) (layer B.Cu) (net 30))
 (segment (start 143.089999 63.920001) (end 142.24 64.77) (width 0.25) (layer B.Cu) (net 30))
 (segment (start 171.544999 65.945001) (end 146.755999 65.945001) (width 0.25) (layer B.Cu) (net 30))
 (segment (start 172.72 64.77) (end 171.544999 65.945001) (width 0.25) (layer B.Cu) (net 30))
 (segment (start 111.74 85.09) (end 114.450002 85.09) (width 0.25) (layer B.Cu) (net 27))
 (segment (start 139.8564 59.683602) (end 140.181402 59.3586) (width 0.25) (layer B.Cu) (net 27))
 (segment (start 138.041396 59.683602) (end 139.8564 59.683602) (width 0.25) (layer B.Cu) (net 27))
 (segment (start 140.181402 59.3586) (end 141.045001 58.495001) (width 0.25) (layer B.Cu) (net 27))
 (segment (start 114.450002 83.274996) (end 138.041396 59.683602) (width 0.25) (layer B.Cu) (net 27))
 (segment (start 114.450002 85.09) (end 114.450002 83.274996) (width 0.25) (layer B.Cu) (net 27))
 (segment (start 135.89 77.47) (end 139.7 81.28) (width 0.25) (layer B.Cu) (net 92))
 (segment (start 133.35 74.93) (end 139.7 81.28) (width 0.25) (layer B.Cu) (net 92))
 (segment (start 132.08 74.93) (end 133.35 74.93) (width 0.25) (layer B.Cu) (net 92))
 (segment (start 143.51 58.570002) (end 143.585001 58.495001) (width 0.25) (layer B.Cu) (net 26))
 (segment (start 134.770002 67.31) (end 132.08 67.31) (width 0.25) (layer B.Cu) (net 26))
 (segment (start 143.585001 58.495001) (end 134.770002 67.31) (width 0.25) (layer B.Cu) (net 26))
 (segment (start 149.86 59.840002) (end 151.205001 58.495001) (width 0.25) (layer B.Cu) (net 23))
 (segment (start 149.86 64.77) (end 149.86 59.840002) (width 0.25) (layer B.Cu) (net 23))
 (segment (start 152.5564 57.3064) (end 152.881402 57.631402) (width 0.25) (layer B.Cu) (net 22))
 (segment (start 152.881402 57.631402) (end 153.745001 58.495001) (width 0.25) (layer B.Cu) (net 22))
 (segment (start 147.32 58.080872) (end 148.094472 57.3064) (width 0.25) (layer B.Cu) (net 22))
 (segment (start 148.094472 57.3064) (end 152.5564 57.3064) (width 0.25) (layer B.Cu) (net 22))
 (segment (start 147.32 64.77) (end 147.32 58.080872) (width 0.25) (layer B.Cu) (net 22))
 (segment (start 139.3686 57.631402) (end 138.505001 58.495001) (width 0.25) (layer B.Cu) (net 28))
 (segment (start 140.143611 56.856391) (end 139.3686 57.631402) (width 0.25) (layer B.Cu) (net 28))
 (segment (start 174.185521 56.856391) (end 140.143611 56.856391) (width 0.25) (layer B.Cu) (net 28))
 (segment (start 175.253602 57.924472) (end 174.185521 56.856391) (width 0.25) (layer B.Cu) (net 28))
 (segment (start 175.253602 72.396398) (end 175.253602 57.924472) (width 0.25) (layer B.Cu) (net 28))
 (segment (start 172.72 74.93) (end 175.253602 72.396398) (width 0.25) (layer B.Cu) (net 28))
 (segment (start 169.8486 57.631402) (end 168.985001 58.495001) (width 0.25) (layer B.Cu) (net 17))
 (segment (start 172.09553 57.3064) (end 170.173602 57.3064) (width 0.25) (layer B.Cu) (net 17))
 (segment (start 172.713602 57.924472) (end 172.09553 57.3064) (width 0.25) (layer B.Cu) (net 17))
 (segment (start 172.713602 59.047192) (end 172.713602 57.924472) (width 0.25) (layer B.Cu) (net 17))
 (segment (start 174.34501 60.6786) (end 172.713602 59.047192) (width 0.25) (layer B.Cu) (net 17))
 (segment (start 174.34501 70.76499) (end 174.34501 60.6786) (width 0.25) (layer B.Cu) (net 17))
 (segment (start 170.173602 57.3064) (end 169.8486 57.631402) (width 0.25) (layer B.Cu) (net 17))
 (segment (start 172.72 72.39) (end 174.34501 70.76499) (width 0.25) (layer B.Cu) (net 17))
 (segment (start 173.895001 60.865001) (end 172.3886 59.3586) (width 0.25) (layer B.Cu) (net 16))
 (segment (start 173.895001 68.674999) (end 173.895001 60.865001) (width 0.25) (layer B.Cu) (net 16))
 (segment (start 172.3886 59.3586) (end 171.525001 58.495001) (width 0.25) (layer B.Cu) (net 16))
 (segment (start 172.72 69.85) (end 173.895001 68.674999) (width 0.25) (layer B.Cu) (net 16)))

